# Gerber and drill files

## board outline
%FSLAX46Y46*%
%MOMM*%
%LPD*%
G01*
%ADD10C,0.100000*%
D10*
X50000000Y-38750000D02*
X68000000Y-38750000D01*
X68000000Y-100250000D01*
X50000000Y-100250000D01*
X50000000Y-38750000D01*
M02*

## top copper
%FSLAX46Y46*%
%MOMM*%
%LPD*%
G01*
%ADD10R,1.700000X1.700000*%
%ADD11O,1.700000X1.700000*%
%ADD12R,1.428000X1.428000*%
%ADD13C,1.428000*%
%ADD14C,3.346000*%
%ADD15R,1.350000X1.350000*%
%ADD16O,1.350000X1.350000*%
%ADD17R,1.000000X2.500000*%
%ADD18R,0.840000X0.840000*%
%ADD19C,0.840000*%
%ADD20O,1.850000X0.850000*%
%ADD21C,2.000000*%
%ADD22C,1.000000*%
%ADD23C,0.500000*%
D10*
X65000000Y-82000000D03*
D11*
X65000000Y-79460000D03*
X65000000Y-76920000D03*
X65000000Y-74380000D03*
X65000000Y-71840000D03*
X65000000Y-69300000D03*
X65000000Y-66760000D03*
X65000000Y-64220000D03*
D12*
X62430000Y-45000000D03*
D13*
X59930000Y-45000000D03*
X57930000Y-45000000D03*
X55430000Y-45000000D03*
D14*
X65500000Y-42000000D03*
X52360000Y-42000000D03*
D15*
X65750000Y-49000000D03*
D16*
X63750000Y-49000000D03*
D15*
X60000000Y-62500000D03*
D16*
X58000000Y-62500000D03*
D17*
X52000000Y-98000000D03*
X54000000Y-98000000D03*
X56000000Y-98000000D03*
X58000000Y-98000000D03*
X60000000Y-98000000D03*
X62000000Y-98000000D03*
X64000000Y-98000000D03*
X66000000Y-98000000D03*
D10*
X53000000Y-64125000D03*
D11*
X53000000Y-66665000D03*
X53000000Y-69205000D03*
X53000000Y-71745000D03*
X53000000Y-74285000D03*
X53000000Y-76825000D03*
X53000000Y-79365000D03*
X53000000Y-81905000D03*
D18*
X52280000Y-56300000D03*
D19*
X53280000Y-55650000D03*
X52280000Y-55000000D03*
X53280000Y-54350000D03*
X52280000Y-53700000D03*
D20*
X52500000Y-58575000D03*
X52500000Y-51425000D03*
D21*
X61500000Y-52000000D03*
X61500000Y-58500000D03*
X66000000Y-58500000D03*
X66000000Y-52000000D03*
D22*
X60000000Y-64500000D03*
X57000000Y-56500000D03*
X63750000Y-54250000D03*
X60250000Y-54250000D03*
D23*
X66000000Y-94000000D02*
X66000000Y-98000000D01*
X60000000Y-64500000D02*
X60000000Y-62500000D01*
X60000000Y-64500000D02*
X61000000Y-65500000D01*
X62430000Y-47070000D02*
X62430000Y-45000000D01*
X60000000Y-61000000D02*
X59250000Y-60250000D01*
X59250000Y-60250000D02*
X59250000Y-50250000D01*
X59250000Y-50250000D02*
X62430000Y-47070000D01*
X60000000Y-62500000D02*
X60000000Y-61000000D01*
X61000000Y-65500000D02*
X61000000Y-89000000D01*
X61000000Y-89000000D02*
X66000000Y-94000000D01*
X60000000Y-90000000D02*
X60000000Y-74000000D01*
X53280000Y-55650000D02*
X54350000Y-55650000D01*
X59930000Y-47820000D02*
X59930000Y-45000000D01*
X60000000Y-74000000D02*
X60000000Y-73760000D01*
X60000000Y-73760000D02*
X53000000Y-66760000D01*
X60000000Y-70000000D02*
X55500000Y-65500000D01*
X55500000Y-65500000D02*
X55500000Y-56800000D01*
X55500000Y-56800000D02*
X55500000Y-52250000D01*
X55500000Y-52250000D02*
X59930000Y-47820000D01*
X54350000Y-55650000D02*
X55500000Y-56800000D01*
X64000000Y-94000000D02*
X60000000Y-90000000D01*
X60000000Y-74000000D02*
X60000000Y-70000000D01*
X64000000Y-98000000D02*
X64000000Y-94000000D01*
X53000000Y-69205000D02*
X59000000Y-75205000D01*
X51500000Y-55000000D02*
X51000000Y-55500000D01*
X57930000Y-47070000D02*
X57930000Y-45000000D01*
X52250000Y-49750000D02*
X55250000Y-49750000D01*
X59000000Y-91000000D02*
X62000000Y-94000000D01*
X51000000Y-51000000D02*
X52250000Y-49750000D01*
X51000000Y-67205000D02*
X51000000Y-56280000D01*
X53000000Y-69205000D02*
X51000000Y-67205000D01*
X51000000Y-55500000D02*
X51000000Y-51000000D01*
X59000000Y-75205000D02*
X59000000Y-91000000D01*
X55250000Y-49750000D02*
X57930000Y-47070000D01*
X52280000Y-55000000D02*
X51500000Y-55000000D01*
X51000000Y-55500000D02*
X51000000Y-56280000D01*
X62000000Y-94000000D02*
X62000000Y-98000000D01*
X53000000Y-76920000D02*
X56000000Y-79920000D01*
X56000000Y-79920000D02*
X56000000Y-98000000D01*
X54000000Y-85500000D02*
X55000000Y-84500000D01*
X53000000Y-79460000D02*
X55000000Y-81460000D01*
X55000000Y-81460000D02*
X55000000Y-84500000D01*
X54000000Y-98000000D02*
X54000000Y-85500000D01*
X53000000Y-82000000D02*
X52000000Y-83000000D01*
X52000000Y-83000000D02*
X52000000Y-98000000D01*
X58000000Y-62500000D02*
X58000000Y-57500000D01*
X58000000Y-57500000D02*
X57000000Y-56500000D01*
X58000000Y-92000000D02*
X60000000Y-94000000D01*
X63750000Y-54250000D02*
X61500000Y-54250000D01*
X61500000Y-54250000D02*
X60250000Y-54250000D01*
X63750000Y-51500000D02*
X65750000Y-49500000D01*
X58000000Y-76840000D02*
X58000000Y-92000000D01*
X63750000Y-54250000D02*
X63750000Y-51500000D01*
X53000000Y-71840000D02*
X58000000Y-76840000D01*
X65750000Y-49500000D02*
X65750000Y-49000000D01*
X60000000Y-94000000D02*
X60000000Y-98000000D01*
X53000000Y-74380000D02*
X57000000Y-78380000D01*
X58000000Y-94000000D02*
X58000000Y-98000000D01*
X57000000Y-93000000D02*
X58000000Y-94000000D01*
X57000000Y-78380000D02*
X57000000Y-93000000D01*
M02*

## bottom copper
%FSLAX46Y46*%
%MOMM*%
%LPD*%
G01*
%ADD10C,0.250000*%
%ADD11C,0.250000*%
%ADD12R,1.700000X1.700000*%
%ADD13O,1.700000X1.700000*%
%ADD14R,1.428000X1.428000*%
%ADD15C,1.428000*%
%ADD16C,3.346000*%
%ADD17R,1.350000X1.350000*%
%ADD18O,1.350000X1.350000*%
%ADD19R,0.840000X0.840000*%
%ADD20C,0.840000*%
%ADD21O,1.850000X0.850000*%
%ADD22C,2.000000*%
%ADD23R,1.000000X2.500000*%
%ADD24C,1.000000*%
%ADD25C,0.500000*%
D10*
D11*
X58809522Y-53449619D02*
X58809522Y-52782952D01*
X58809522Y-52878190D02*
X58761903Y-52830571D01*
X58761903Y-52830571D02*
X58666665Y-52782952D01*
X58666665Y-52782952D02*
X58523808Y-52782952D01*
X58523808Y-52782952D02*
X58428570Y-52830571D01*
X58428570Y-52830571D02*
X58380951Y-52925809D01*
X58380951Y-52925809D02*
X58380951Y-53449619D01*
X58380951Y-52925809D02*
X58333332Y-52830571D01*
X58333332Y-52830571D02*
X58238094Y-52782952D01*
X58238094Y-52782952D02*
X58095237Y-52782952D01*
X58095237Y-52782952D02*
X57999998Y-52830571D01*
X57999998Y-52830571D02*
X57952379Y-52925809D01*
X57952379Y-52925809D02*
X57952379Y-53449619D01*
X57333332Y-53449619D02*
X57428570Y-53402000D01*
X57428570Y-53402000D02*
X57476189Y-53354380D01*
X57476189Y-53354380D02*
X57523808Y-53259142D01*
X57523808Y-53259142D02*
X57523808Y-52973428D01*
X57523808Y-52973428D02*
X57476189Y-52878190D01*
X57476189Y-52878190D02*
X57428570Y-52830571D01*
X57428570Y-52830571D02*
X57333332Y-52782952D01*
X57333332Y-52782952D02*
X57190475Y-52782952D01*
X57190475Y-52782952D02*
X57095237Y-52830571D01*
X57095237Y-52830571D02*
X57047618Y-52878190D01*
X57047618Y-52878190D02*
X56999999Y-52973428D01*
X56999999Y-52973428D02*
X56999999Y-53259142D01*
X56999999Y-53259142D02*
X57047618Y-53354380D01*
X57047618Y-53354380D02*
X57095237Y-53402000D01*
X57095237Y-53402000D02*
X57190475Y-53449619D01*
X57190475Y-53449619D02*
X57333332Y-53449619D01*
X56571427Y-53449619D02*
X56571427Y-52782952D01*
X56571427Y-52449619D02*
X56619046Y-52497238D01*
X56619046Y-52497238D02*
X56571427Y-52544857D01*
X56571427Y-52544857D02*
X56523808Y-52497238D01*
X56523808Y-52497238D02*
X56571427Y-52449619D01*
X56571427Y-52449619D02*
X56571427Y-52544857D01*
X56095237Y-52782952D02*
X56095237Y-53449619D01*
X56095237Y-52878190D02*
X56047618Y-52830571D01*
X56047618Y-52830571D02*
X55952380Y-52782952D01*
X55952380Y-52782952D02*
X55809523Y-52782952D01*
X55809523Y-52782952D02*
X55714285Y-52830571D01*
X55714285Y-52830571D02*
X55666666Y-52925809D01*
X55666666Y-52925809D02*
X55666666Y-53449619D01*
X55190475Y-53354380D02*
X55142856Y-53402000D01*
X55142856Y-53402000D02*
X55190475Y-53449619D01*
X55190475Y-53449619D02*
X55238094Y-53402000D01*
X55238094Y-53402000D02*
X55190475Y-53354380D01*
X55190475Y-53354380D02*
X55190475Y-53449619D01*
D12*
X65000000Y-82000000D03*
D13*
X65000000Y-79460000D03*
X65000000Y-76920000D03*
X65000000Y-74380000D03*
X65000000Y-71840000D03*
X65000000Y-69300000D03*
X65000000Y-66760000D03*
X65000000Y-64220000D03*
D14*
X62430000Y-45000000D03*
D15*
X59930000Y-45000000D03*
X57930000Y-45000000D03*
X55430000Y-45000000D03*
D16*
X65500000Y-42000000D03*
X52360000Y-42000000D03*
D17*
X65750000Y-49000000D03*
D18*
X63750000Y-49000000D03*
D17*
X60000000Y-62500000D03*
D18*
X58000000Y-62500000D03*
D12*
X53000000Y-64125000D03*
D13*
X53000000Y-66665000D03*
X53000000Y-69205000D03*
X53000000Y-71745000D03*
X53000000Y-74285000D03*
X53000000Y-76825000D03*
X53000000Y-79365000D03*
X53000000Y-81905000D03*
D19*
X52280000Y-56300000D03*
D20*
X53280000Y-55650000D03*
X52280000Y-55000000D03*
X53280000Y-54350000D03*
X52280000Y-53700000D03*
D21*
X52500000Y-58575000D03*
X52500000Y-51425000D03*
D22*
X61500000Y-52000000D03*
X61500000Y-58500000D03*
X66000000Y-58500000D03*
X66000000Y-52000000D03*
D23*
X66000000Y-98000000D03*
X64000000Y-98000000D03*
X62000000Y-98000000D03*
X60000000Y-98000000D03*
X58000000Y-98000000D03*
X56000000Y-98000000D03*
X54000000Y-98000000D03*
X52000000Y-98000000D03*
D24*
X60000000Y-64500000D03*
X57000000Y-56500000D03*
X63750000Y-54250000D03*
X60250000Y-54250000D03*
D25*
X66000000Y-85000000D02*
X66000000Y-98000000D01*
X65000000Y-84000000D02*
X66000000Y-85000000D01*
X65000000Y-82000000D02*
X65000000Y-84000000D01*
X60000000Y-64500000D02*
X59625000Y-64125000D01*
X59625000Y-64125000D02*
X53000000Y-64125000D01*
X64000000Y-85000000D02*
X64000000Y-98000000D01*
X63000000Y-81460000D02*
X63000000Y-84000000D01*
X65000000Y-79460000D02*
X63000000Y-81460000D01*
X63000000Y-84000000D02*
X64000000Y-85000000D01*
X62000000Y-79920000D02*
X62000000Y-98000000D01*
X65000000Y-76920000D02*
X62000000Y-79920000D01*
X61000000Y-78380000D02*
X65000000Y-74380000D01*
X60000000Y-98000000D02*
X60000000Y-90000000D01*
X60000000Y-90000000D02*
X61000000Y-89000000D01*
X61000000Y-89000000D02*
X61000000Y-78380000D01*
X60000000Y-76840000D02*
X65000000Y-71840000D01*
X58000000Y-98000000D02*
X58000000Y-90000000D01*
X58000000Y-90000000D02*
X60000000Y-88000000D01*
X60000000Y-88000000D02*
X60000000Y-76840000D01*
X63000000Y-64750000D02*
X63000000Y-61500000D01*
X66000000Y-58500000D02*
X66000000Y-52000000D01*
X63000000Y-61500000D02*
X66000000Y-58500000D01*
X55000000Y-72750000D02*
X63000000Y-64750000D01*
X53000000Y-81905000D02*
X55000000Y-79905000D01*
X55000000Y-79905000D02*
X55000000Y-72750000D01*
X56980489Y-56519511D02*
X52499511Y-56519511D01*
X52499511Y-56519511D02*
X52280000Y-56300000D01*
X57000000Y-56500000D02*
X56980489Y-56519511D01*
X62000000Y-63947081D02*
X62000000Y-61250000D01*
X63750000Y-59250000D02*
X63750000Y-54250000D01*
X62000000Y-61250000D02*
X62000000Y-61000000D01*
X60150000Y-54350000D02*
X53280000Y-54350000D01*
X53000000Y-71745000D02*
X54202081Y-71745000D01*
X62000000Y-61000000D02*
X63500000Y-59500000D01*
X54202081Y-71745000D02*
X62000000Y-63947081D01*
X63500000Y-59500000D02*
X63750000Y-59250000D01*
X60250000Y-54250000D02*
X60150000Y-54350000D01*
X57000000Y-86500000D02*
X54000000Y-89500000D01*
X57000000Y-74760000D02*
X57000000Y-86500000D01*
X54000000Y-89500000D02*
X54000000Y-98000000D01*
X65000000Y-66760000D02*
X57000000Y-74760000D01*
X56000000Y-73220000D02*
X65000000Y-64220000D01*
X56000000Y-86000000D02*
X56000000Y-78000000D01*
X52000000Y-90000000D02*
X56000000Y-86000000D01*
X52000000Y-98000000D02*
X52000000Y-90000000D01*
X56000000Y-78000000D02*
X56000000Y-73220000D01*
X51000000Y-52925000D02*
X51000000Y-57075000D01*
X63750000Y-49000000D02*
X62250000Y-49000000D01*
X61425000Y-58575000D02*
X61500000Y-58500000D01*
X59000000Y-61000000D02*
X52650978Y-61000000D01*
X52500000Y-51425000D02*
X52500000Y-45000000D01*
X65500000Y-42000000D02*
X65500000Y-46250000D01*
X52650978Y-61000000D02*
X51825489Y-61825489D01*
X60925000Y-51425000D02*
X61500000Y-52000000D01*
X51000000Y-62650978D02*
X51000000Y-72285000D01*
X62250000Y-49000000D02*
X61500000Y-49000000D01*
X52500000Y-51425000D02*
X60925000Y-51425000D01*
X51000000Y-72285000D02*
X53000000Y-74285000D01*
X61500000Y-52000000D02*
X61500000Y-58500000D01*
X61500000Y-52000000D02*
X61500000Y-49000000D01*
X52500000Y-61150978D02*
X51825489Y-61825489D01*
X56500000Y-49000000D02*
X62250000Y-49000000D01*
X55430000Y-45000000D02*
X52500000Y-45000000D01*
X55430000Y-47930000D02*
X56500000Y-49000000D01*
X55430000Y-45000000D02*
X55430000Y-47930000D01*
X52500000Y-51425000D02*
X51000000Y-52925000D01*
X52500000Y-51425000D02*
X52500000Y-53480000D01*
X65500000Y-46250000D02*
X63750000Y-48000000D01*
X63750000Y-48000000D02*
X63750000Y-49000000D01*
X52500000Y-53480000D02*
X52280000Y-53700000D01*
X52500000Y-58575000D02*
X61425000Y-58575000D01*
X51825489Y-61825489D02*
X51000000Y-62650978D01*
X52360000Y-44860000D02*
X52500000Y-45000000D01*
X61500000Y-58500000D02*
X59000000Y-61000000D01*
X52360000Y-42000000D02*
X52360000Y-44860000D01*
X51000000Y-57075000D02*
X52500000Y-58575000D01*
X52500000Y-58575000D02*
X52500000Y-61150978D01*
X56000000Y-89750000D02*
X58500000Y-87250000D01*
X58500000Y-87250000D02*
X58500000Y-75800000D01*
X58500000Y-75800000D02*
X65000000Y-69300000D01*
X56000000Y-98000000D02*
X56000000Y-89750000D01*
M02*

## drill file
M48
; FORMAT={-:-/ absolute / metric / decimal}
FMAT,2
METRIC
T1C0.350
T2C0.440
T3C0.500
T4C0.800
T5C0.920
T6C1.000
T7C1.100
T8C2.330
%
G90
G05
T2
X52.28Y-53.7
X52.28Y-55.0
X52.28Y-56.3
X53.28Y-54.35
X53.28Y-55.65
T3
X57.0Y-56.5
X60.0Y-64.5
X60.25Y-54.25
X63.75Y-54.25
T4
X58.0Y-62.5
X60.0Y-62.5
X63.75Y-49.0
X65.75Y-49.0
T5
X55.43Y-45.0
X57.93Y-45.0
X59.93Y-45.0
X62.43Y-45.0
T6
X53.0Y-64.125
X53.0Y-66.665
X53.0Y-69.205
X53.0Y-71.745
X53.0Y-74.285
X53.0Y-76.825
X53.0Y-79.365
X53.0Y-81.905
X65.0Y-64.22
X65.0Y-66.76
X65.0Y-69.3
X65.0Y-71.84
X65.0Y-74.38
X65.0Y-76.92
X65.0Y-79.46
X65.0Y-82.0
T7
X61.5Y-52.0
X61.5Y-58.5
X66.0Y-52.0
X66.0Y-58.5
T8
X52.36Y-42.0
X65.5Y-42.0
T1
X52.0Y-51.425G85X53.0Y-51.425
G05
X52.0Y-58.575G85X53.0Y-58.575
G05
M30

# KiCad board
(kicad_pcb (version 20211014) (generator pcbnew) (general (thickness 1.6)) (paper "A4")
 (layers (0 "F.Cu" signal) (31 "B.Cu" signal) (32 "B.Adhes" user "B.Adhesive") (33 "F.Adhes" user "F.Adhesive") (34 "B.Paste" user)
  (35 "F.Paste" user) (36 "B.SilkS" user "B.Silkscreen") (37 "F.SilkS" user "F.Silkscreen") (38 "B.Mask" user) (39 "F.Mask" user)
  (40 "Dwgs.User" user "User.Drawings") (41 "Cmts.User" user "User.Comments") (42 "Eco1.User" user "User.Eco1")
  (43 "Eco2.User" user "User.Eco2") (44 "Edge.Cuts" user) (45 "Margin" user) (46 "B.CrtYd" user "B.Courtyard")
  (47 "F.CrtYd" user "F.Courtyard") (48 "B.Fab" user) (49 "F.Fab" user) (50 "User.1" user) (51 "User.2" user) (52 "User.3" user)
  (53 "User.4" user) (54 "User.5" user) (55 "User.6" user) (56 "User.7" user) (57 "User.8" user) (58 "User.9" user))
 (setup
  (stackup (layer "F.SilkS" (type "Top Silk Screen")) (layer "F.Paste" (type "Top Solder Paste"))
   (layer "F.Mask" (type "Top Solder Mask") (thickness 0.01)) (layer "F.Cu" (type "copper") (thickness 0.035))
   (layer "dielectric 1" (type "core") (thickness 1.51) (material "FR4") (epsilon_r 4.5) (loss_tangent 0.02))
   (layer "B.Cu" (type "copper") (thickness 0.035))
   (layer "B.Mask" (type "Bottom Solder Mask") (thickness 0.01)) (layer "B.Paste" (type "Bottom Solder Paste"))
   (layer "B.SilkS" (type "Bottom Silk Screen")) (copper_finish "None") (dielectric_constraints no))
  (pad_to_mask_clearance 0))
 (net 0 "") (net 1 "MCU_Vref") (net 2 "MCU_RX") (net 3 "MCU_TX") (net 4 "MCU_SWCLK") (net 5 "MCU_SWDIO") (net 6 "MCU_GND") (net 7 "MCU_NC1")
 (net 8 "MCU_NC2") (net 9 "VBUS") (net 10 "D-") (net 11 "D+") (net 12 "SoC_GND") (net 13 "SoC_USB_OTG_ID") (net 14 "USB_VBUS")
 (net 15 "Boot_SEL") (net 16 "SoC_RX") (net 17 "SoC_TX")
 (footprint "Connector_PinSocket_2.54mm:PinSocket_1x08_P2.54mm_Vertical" (layer "F.Cu") (at 65 82 180)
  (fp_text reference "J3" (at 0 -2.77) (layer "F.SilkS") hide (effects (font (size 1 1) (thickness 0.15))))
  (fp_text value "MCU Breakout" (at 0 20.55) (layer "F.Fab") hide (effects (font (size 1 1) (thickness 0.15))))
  (pad "1" thru_hole rect (at 0 0 180) (size 1.7 1.7) (drill 1) (layers *.Cu *.Mask) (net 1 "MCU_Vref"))
  (pad "2" thru_hole oval (at 0 2.54 180) (size 1.7 1.7) (drill 1) (layers *.Cu *.Mask) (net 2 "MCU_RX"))
  (pad "3" thru_hole oval (at 0 5.08 180) (size 1.7 1.7) (drill 1) (layers *.Cu *.Mask) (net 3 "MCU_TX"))
  (pad "4" thru_hole oval (at 0 7.62 180) (size 1.7 1.7) (drill 1) (layers *.Cu *.Mask) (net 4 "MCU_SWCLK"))
  (pad "5" thru_hole oval (at 0 10.16 180) (size 1.7 1.7) (drill 1) (layers *.Cu *.Mask) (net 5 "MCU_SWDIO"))
  (pad "6" thru_hole oval (at 0 12.7 180) (size 1.7 1.7) (drill 1) (layers *.Cu *.Mask) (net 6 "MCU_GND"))
  (pad "7" thru_hole oval (at 0 15.24 180) (size 1.7 1.7) (drill 1) (layers *.Cu *.Mask) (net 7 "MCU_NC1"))
  (pad "8" thru_hole oval (at 0 17.78 180) (size 1.7 1.7) (drill 1) (layers *.Cu *.Mask) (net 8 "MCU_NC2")))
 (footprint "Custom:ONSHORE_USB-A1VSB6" (layer "F.Cu") (at 58.93 42 180)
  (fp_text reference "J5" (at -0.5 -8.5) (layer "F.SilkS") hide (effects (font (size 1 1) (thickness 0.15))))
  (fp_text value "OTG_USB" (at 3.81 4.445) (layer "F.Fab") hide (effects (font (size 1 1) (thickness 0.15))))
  (pad "1" thru_hole rect (at -3.5 -3 180) (size 1.428 1.428) (drill 0.92) (layers *.Cu *.Mask) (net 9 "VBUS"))
  (pad "2" thru_hole circle (at -1 -3 180) (size 1.428 1.428) (drill 0.92) (layers *.Cu *.Mask) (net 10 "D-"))
  (pad "3" thru_hole circle (at 1 -3 180) (size 1.428 1.428) (drill 0.92) (layers *.Cu *.Mask) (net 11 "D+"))
  (pad "4" thru_hole circle (at 3.5 -3 180) (size 1.428 1.428) (drill 0.92) (layers *.Cu *.Mask) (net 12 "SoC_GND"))
  (pad "S1" thru_hole circle (at -6.57 0 180) (size 3.346 3.346) (drill 2.33) (layers *.Cu *.Mask) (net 12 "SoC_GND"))
  (pad "S2" thru_hole circle (at 6.57 0 180) (size 3.346 3.346) (drill 2.33) (layers *.Cu *.Mask) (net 12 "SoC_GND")))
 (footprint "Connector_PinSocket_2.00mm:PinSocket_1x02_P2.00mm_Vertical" (layer "F.Cu") (at 65.75 49 -90)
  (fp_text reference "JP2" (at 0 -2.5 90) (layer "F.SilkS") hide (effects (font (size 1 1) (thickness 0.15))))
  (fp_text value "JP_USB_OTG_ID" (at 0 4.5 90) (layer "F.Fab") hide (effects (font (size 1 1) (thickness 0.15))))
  (pad "1" thru_hole rect (at 0 0 270) (size 1.35 1.35) (drill 0.8) (layers *.Cu *.Mask) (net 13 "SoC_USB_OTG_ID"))
  (pad "2" thru_hole oval (at 0 2 270) (size 1.35 1.35) (drill 0.8) (layers *.Cu *.Mask) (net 12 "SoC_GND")))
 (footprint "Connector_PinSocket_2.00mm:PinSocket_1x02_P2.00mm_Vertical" (layer "F.Cu") (at 60 62.5 -90)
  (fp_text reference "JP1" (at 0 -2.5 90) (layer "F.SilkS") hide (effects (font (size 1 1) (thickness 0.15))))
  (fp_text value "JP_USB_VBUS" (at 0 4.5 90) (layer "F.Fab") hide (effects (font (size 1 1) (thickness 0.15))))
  (pad "1" thru_hole rect (at 0 0 270) (size 1.35 1.35) (drill 0.8) (layers *.Cu *.Mask) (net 9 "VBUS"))
  (pad "2" thru_hole oval (at 0 2 270) (size 1.35 1.35) (drill 0.8) (layers *.Cu *.Mask) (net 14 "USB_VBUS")))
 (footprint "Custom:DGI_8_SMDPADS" (layer "F.Cu") (at 59 98)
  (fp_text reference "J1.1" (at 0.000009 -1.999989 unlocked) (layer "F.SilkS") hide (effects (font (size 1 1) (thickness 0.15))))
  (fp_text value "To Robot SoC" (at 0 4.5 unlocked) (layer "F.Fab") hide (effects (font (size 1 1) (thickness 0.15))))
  (pad "1" smd rect (at -7 0) (size 1 2.5) (layers "F.Cu" "F.Paste" "F.Mask") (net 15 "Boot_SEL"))
  (pad "2" smd rect (at -5 0) (size 1 2.5) (layers "F.Cu" "F.Paste" "F.Mask") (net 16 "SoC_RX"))
  (pad "3" smd rect (at -3 0) (size 1 2.5) (layers "F.Cu" "F.Paste" "F.Mask") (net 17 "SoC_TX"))
  (pad "4" smd rect (at -1 0) (size 1 2.5) (layers "F.Cu" "F.Paste" "F.Mask") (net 12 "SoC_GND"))
  (pad "5" smd rect (at 1 0) (size 1 2.5) (layers "F.Cu" "F.Paste" "F.Mask") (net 13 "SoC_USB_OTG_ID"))
  (pad "6" smd rect (at 3 0) (size 1 2.5) (layers "F.Cu" "F.Paste" "F.Mask") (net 11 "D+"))
  (pad "7" smd rect (at 5 0) (size 1 2.5) (layers "F.Cu" "F.Paste" "F.Mask") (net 10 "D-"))
  (pad "8" smd rect (at 7 0) (size 1 2.5) (layers "F.Cu" "F.Paste" "F.Mask") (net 9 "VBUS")))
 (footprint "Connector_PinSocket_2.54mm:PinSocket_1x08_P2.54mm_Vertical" (layer "F.Cu") (at 53 64.125)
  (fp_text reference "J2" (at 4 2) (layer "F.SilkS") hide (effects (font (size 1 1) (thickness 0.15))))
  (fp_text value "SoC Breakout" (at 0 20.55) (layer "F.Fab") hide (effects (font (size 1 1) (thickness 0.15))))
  (pad "1" thru_hole rect (at 0 0) (size 1.7 1.7) (drill 1) (layers *.Cu *.Mask) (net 9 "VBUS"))
  (pad "2" thru_hole oval (at 0 2.54) (size 1.7 1.7) (drill 1) (layers *.Cu *.Mask) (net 10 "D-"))
  (pad "3" thru_hole oval (at 0 5.08) (size 1.7 1.7) (drill 1) (layers *.Cu *.Mask) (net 11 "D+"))
  (pad "4" thru_hole oval (at 0 7.62) (size 1.7 1.7) (drill 1) (layers *.Cu *.Mask) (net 13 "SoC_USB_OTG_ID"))
  (pad "5" thru_hole oval (at 0 10.16) (size 1.7 1.7) (drill 1) (layers *.Cu *.Mask) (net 12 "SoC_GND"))
  (pad "6" thru_hole oval (at 0 12.7) (size 1.7 1.7) (drill 1) (layers *.Cu *.Mask) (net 17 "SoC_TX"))
  (pad "7" thru_hole oval (at 0 15.24) (size 1.7 1.7) (drill 1) (layers *.Cu *.Mask) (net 16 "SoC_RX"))
  (pad "8" thru_hole oval (at 0 17.78) (size 1.7 1.7) (drill 1) (layers *.Cu *.Mask) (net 15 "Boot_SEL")))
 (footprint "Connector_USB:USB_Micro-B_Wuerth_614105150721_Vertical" (layer "F.Cu") (at 52.28 56.3 90)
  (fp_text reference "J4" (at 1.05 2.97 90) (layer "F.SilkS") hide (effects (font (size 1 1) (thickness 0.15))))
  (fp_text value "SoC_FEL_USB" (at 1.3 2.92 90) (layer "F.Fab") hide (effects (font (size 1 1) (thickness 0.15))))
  (pad "1" thru_hole rect (at 0 0 90) (size 0.84 0.84) (drill 0.44) (layers *.Cu *.Mask) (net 14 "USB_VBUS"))
  (pad "2" thru_hole circle (at 0.65 1 90) (size 0.84 0.84) (drill 0.44) (layers *.Cu *.Mask) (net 10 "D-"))
  (pad "3" thru_hole circle (at 1.3 0 90) (size 0.84 0.84) (drill 0.44) (layers *.Cu *.Mask) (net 11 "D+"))
  (pad "4" thru_hole circle (at 1.95 1 90) (size 0.84 0.84) (drill 0.44) (layers *.Cu *.Mask) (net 13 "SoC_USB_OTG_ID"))
  (pad "5" thru_hole circle (at 2.6 0 90) (size 0.84 0.84) (drill 0.44) (layers *.Cu *.Mask) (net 12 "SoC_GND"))
  (pad "6" thru_hole oval (at -2.275 0.22 90) (size 0.85 1.85) (drill oval 0.35 1.35) (layers *.Cu *.Mask) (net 12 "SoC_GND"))
  (pad "6" thru_hole oval (at 4.875 0.22 90) (size 0.85 1.85) (drill oval 0.35 1.35) (layers *.Cu *.Mask) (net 12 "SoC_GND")))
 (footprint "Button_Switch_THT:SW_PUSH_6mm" (layer "F.Cu") (at 61.5 58.5 90)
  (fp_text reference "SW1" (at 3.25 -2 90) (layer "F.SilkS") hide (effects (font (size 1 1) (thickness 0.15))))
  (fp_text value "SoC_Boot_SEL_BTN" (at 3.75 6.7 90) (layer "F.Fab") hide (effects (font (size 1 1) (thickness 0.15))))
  (pad "1" thru_hole circle (at 6.5 0 180) (size 2 2) (drill 1.1) (layers *.Cu *.Mask) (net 12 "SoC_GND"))
  (pad "1" thru_hole circle (at 0 0 180) (size 2 2) (drill 1.1) (layers *.Cu *.Mask) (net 12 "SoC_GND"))
  (pad "2" thru_hole circle (at 0 4.5 180) (size 2 2) (drill 1.1) (layers *.Cu *.Mask) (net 15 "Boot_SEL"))
  (pad "2" thru_hole circle (at 6.5 4.5 180) (size 2 2) (drill 1.1) (layers *.Cu *.Mask) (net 15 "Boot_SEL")))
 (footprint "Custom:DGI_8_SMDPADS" (layer "B.Cu") (at 59 98 180)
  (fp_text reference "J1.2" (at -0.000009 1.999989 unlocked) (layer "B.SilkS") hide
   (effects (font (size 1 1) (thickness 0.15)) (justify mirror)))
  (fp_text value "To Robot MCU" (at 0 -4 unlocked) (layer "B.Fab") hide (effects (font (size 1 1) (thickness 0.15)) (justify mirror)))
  (pad "1" smd rect (at -7 0 180) (size 1 2.5) (layers "B.Cu" "B.Paste" "B.Mask") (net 1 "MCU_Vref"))
  (pad "2" smd rect (at -5 0 180) (size 1 2.5) (layers "B.Cu" "B.Paste" "B.Mask") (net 2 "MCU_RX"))
  (pad "3" smd rect (at -3 0 180) (size 1 2.5) (layers "B.Cu" "B.Paste" "B.Mask") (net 3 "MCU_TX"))
  (pad "4" smd rect (at -1 0 180) (size 1 2.5) (layers "B.Cu" "B.Paste" "B.Mask") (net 4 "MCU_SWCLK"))
  (pad "5" smd rect (at 1 0 180) (size 1 2.5) (layers "B.Cu" "B.Paste" "B.Mask") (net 5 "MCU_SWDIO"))
  (pad "6" smd rect (at 3 0 180) (size 1 2.5) (layers "B.Cu" "B.Paste" "B.Mask") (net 6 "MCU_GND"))
  (pad "7" smd rect (at 5 0 180) (size 1 2.5) (layers "B.Cu" "B.Paste" "B.Mask") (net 7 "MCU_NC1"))
  (pad "8" smd rect (at 7 0 180) (size 1 2.5) (layers "B.Cu" "B.Paste" "B.Mask") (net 8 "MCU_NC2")))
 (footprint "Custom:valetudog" (layer "B.Cu") (at 59 80.25 180)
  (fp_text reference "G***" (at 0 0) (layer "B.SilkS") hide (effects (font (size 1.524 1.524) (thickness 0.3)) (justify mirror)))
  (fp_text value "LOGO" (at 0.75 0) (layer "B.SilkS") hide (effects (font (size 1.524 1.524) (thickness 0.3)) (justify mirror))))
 (gr_rect (start 50 100.25) (end 68 38.75) (layer "Edge.Cuts") (width 0.1) (fill none))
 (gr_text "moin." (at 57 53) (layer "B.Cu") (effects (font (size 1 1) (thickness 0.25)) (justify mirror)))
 (segment (start 66 85) (end 66 98) (width 0.5) (layer "B.Cu") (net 1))
 (segment (start 65 84) (end 66 85) (width 0.5) (layer "B.Cu") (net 1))
 (segment (start 65 82) (end 65 84) (width 0.5) (layer "B.Cu") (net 1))
 (segment (start 66 94) (end 66 98) (width 0.5) (layer "F.Cu") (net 9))
 (segment (start 60 64.5) (end 60 62.5) (width 0.5) (layer "F.Cu") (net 9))
 (segment (start 60 64.5) (end 61 65.5) (width 0.5) (layer "F.Cu") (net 9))
 (segment (start 62.43 47.07) (end 62.43 45) (width 0.5) (layer "F.Cu") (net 9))
 (segment (start 60 61) (end 59.25 60.25) (width 0.5) (layer "F.Cu") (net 9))
 (segment (start 59.25 60.25) (end 59.25 50.25) (width 0.5) (layer "F.Cu") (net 9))
 (segment (start 59.25 50.25) (end 62.43 47.07) (width 0.5) (layer "F.Cu") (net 9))
 (segment (start 60 62.5) (end 60 61) (width 0.5) (layer "F.Cu") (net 9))
 (segment (start 61 65.5) (end 61 89) (width 0.5) (layer "F.Cu") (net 9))
 (segment (start 61 89) (end 66 94) (width 0.5) (layer "F.Cu") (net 9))
 (via (at 60 64.5) (size 1) (drill 0.5) (layers "F.Cu" "B.Cu") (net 9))
 (segment (start 60 64.5) (end 59.625 64.125) (width 0.5) (layer "B.Cu") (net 9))
 (segment (start 59.625 64.125) (end 53 64.125) (width 0.5) (layer "B.Cu") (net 9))
 (segment (start 64 85) (end 64 98) (width 0.5) (layer "B.Cu") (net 2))
 (segment (start 63 81.46) (end 63 84) (width 0.5) (layer "B.Cu") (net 2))
 (segment (start 65 79.46) (end 63 81.46) (width 0.5) (layer "B.Cu") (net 2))
 (segment (start 63 84) (end 64 85) (width 0.5) (layer "B.Cu") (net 2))
 (segment (start 60 90) (end 60 74) (width 0.5) (layer "F.Cu") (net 10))
 (segment (start 53.28 55.65) (end 54.35 55.65) (width 0.5) (layer "F.Cu") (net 10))
 (segment (start 59.93 47.82) (end 59.93 45) (width 0.5) (layer "F.Cu") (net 10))
 (segment (start 60 74) (end 60 73.76) (width 0.5) (layer "F.Cu") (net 10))
 (segment (start 60 73.76) (end 53 66.76) (width 0.5) (layer "F.Cu") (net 10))
 (segment (start 60 70) (end 55.5 65.5) (width 0.5) (layer "F.Cu") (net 10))
 (segment (start 55.5 65.5) (end 55.5 56.8) (width 0.5) (layer "F.Cu") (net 10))
 (segment (start 55.5 56.8) (end 55.5 52.25) (width 0.5) (layer "F.Cu") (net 10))
 (segment (start 55.5 52.25) (end 59.93 47.82) (width 0.5) (layer "F.Cu") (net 10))
 (segment (start 54.35 55.65) (end 55.5 56.8) (width 0.5) (layer "F.Cu") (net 10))
 (segment (start 64 94) (end 60 90) (width 0.5) (layer "F.Cu") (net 10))
 (segment (start 60 74) (end 60 70) (width 0.5) (layer "F.Cu") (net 10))
 (segment (start 64 98) (end 64 94) (width 0.5) (layer "F.Cu") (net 10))
 (segment (start 62 79.92) (end 62 98) (width 0.5) (layer "B.Cu") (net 3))
 (segment (start 65 76.92) (end 62 79.92) (width 0.5) (layer "B.Cu") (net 3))
 (segment (start 53 69.205) (end 59 75.205) (width 0.5) (layer "F.Cu") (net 11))
 (segment (start 51.5 55) (end 51 55.5) (width 0.5) (layer "F.Cu") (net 11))
 (segment (start 57.93 47.07) (end 57.93 45) (width 0.5) (layer "F.Cu") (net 11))
 (segment (start 52.25 49.75) (end 55.25 49.75) (width 0.5) (layer "F.Cu") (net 11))
 (segment (start 59 91) (end 62 94) (width 0.5) (layer "F.Cu") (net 11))
 (segment (start 51 51) (end 52.25 49.75) (width 0.5) (layer "F.Cu") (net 11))
 (segment (start 51 67.205) (end 51 56.28) (width 0.5) (layer "F.Cu") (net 11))
 (segment (start 53 69.205) (end 51 67.205) (width 0.5) (layer "F.Cu") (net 11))
 (segment (start 51 55.5) (end 51 51) (width 0.5) (layer "F.Cu") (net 11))
 (segment (start 59 75.205) (end 59 91) (width 0.5) (layer "F.Cu") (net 11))
 (segment (start 55.25 49.75) (end 57.93 47.07) (width 0.5) (layer "F.Cu") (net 11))
 (segment (start 52.28 55) (end 51.5 55) (width 0.5) (layer "F.Cu") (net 11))
 (segment (start 51 55.5) (end 51 56.28) (width 0.5) (layer "F.Cu") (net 11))
 (segment (start 62 94) (end 62 98) (width 0.5) (layer "F.Cu") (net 11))
 (segment (start 61 78.38) (end 65 74.38) (width 0.5) (layer "B.Cu") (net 4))
 (segment (start 60 98) (end 60 90) (width 0.5) (layer "B.Cu") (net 4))
 (segment (start 60 90) (end 61 89) (width 0.5) (layer "B.Cu") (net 4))
 (segment (start 61 89) (end 61 78.38) (width 0.5) (layer "B.Cu") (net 4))
 (segment (start 60 76.84) (end 65 71.84) (width 0.5) (layer "B.Cu") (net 5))
 (segment (start 58 98) (end 58 90) (width 0.5) (layer "B.Cu") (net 5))
 (segment (start 58 90) (end 60 88) (width 0.5) (layer "B.Cu") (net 5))
 (segment (start 60 88) (end 60 76.84) (width 0.5) (layer "B.Cu") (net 5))
 (segment (start 53 76.92) (end 56 79.92) (width 0.5) (layer "F.Cu") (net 17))
 (segment (start 56 79.92) (end 56 98) (width 0.5) (layer "F.Cu") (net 17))
 (segment (start 54 85.5) (end 55 84.5) (width 0.5) (layer "F.Cu") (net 16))
 (segment (start 53 79.46) (end 55 81.46) (width 0.5) (layer "F.Cu") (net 16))
 (segment (start 55 81.46) (end 55 84.5) (width 0.5) (layer "F.Cu") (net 16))
 (segment (start 54 98) (end 54 85.5) (width 0.5) (layer "F.Cu") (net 16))
 (segment (start 53 82) (end 52 83) (width 0.5) (layer "F.Cu") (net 15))
 (segment (start 52 83) (end 52 98) (width 0.5) (layer "F.Cu") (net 15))
 (segment (start 63 64.75) (end 63 61.5) (width 0.5) (layer "B.Cu") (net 15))
 (segment (start 66 58.5) (end 66 52) (width 0.5) (layer "B.Cu") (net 15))
 (segment (start 63 61.5) (end 66 58.5) (width 0.5) (layer "B.Cu") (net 15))
 (segment (start 55 72.75) (end 63 64.75) (width 0.5) (layer "B.Cu") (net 15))
 (segment (start 53 81.905) (end 55 79.905) (width 0.5) (layer "B.Cu") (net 15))
 (segment (start 55 79.905) (end 55 72.75) (width 0.5) (layer "B.Cu") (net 15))
 (segment (start 58 62.5) (end 58 57.5) (width 0.5) (layer "F.Cu") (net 14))
 (segment (start 58 57.5) (end 57 56.5) (width 0.5) (layer "F.Cu") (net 14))
 (via (at 57 56.5) (size 1) (drill 0.5) (layers "F.Cu" "B.Cu") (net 14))
 (segment (start 56.980489 56.519511) (end 52.499511 56.519511) (width 0.5) (layer "B.Cu") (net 14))
 (segment (start 52.499511 56.519511) (end 52.28 56.3) (width 0.5) (layer "B.Cu") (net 14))
 (segment (start 57 56.5) (end 56.980489 56.519511) (width 0.5) (layer "B.Cu") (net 14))
 (segment (start 58 92) (end 60 94) (width 0.5) (layer "F.Cu") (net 13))
 (segment (start 63.75 54.25) (end 61.5 54.25) (width 0.5) (layer "F.Cu") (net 13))
 (segment (start 61.5 54.25) (end 60.25 54.25) (width 0.5) (layer "F.Cu") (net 13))
 (segment (start 63.75 51.5) (end 65.75 49.5) (width 0.5) (layer "F.Cu") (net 13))
 (segment (start 58 76.84) (end 58 92) (width 0.5) (layer "F.Cu") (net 13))
 (segment (start 63.75 54.25) (end 63.75 51.5) (width 0.5) (layer "F.Cu") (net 13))
 (segment (start 53 71.84) (end 58 76.84) (width 0.5) (layer "F.Cu") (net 13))
 (segment (start 65.75 49.5) (end 65.75 49) (width 0.5) (layer "F.Cu") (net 13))
 (segment (start 60 94) (end 60 98) (width 0.5) (layer "F.Cu") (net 13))
 (via (at 63.75 54.25) (size 1) (drill 0.5) (layers "F.Cu" "B.Cu") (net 13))
 (via (at 60.25 54.25) (size 1) (drill 0.5) (layers "F.Cu" "B.Cu") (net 13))
 (segment (start 62 63.947081) (end 62 61.25) (width 0.5) (layer "B.Cu") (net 13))
 (segment (start 63.75 59.25) (end 63.75 54.25) (width 0.5) (layer "B.Cu") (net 13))
 (segment (start 62 61.25) (end 62 61) (width 0.5) (layer "B.Cu") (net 13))
 (segment (start 60.15 54.35) (end 53.28 54.35) (width 0.5) (layer "B.Cu") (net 13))
 (segment (start 53 71.745) (end 54.202081 71.745) (width 0.5) (layer "B.Cu") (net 13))
 (segment (start 62 61) (end 63.5 59.5) (width 0.5) (layer "B.Cu") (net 13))
 (segment (start 54.202081 71.745) (end 62 63.947081) (width 0.5) (layer "B.Cu") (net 13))
 (segment (start 63.5 59.5) (end 63.75 59.25) (width 0.5) (layer "B.Cu") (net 13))
 (segment (start 60.25 54.25) (end 60.15 54.35) (width 0.5) (layer "B.Cu") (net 13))
 (segment (start 57 86.5) (end 54 89.5) (width 0.5) (layer "B.Cu") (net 7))
 (segment (start 57 74.76) (end 57 86.5) (width 0.5) (layer "B.Cu") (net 7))
 (segment (start 54 89.5) (end 54 98) (width 0.5) (layer "B.Cu") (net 7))
 (segment (start 65 66.76) (end 57 74.76) (width 0.5) (layer "B.Cu") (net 7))
 (segment (start 56 73.22) (end 65 64.22) (width 0.5) (layer "B.Cu") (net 8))
 (segment (start 56 86) (end 56 78) (width 0.5) (layer "B.Cu") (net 8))
 (segment (start 52 90) (end 56 86) (width 0.5) (layer "B.Cu") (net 8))
 (segment (start 52 98) (end 52 90) (width 0.5) (layer "B.Cu") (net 8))
 (segment (start 56 78) (end 56 73.22) (width 0.5) (layer "B.Cu") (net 8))
 (segment (start 53 74.38) (end 57 78.38) (width 0.5) (layer "F.Cu") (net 12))
 (segment (start 58 94) (end 58 98) (width 0.5) (layer "F.Cu") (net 12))
 (segment (start 57 93) (end 58 94) (width 0.5) (layer "F.Cu") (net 12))
 (segment (start 57 78.38) (end 57 93) (width 0.5) (layer "F.Cu") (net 12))
 (segment (start 51 52.925) (end 51 57.075) (width 0.5) (layer "B.Cu") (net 12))
 (segment (start 63.75 49) (end 62.25 49) (width 0.5) (layer "B.Cu") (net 12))
 (segment (start 61.425 58.575) (end 61.5 58.5) (width 0.5) (layer "B.Cu") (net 12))
 (segment (start 59 61) (end 52.650978 61) (width 0.5) (layer "B.Cu") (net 12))
 (segment (start 52.5 51.425) (end 52.5 45) (width 0.5) (layer "B.Cu") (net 12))
 (segment (start 65.5 42) (end 65.5 46.25) (width 0.5) (layer "B.Cu") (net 12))
 (segment (start 52.650978 61) (end 51.825489 61.825489) (width 0.5) (layer "B.Cu") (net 12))
 (segment (start 60.925 51.425) (end 61.5 52) (width 0.5) (layer "B.Cu") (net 12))
 (segment (start 51 62.650978) (end 51 72.285) (width 0.5) (layer "B.Cu") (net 12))
 (segment (start 62.25 49) (end 61.5 49) (width 0.5) (layer "B.Cu") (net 12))
 (segment (start 52.5 51.425) (end 60.925 51.425) (width 0.5) (layer "B.Cu") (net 12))
 (segment (start 51 72.285) (end 53 74.285) (width 0.5) (layer "B.Cu") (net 12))
 (segment (start 61.5 52) (end 61.5 58.5) (width 0.5) (layer "B.Cu") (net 12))
 (segment (start 61.5 52) (end 61.5 49) (width 0.5) (layer "B.Cu") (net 12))
 (segment (start 52.5 61.150978) (end 51.825489 61.825489) (width 0.5) (layer "B.Cu") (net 12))
 (segment (start 56.5 49) (end 62.25 49) (width 0.5) (layer "B.Cu") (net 12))
 (segment (start 55.43 45) (end 52.5 45) (width 0.5) (layer "B.Cu") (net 12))
 (segment (start 55.43 47.93) (end 56.5 49) (width 0.5) (layer "B.Cu") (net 12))
 (segment (start 55.43 45) (end 55.43 47.93) (width 0.5) (layer "B.Cu") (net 12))
 (segment (start 52.5 51.425) (end 51 52.925) (width 0.5) (layer "B.Cu") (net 12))
 (segment (start 52.5 51.425) (end 52.5 53.48) (width 0.5) (layer "B.Cu") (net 12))
 (segment (start 65.5 46.25) (end 63.75 48) (width 0.5) (layer "B.Cu") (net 12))
 (segment (start 63.75 48) (end 63.75 49) (width 0.5) (layer "B.Cu") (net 12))
 (segment (start 52.5 53.48) (end 52.28 53.7) (width 0.5) (layer "B.Cu") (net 12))
 (segment (start 52.5 58.575) (end 61.425 58.575) (width 0.5) (layer "B.Cu") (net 12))
 (segment (start 51.825489 61.825489) (end 51 62.650978) (width 0.5) (layer "B.Cu") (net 12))
 (segment (start 52.36 44.86) (end 52.5 45) (width 0.5) (layer "B.Cu") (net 12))
 (segment (start 61.5 58.5) (end 59 61) (width 0.5) (layer "B.Cu") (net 12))
 (segment (start 52.36 42) (end 52.36 44.86) (width 0.5) (layer "B.Cu") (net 12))
 (segment (start 51 57.075) (end 52.5 58.575) (width 0.5) (layer "B.Cu") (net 12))
 (segment (start 52.5 58.575) (end 52.5 61.150978) (width 0.5) (layer "B.Cu") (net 12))
 (segment (start 56 89.75) (end 58.5 87.25) (width 0.5) (layer "B.Cu") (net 6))
 (segment (start 58.5 87.25) (end 58.5 75.8) (width 0.5) (layer "B.Cu") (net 6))
 (segment (start 58.5 75.8) (end 65 69.3) (width 0.5) (layer "B.Cu") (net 6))
 (segment (start 56 98) (end 56 89.75) (width 0.5) (layer "B.Cu") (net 6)))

